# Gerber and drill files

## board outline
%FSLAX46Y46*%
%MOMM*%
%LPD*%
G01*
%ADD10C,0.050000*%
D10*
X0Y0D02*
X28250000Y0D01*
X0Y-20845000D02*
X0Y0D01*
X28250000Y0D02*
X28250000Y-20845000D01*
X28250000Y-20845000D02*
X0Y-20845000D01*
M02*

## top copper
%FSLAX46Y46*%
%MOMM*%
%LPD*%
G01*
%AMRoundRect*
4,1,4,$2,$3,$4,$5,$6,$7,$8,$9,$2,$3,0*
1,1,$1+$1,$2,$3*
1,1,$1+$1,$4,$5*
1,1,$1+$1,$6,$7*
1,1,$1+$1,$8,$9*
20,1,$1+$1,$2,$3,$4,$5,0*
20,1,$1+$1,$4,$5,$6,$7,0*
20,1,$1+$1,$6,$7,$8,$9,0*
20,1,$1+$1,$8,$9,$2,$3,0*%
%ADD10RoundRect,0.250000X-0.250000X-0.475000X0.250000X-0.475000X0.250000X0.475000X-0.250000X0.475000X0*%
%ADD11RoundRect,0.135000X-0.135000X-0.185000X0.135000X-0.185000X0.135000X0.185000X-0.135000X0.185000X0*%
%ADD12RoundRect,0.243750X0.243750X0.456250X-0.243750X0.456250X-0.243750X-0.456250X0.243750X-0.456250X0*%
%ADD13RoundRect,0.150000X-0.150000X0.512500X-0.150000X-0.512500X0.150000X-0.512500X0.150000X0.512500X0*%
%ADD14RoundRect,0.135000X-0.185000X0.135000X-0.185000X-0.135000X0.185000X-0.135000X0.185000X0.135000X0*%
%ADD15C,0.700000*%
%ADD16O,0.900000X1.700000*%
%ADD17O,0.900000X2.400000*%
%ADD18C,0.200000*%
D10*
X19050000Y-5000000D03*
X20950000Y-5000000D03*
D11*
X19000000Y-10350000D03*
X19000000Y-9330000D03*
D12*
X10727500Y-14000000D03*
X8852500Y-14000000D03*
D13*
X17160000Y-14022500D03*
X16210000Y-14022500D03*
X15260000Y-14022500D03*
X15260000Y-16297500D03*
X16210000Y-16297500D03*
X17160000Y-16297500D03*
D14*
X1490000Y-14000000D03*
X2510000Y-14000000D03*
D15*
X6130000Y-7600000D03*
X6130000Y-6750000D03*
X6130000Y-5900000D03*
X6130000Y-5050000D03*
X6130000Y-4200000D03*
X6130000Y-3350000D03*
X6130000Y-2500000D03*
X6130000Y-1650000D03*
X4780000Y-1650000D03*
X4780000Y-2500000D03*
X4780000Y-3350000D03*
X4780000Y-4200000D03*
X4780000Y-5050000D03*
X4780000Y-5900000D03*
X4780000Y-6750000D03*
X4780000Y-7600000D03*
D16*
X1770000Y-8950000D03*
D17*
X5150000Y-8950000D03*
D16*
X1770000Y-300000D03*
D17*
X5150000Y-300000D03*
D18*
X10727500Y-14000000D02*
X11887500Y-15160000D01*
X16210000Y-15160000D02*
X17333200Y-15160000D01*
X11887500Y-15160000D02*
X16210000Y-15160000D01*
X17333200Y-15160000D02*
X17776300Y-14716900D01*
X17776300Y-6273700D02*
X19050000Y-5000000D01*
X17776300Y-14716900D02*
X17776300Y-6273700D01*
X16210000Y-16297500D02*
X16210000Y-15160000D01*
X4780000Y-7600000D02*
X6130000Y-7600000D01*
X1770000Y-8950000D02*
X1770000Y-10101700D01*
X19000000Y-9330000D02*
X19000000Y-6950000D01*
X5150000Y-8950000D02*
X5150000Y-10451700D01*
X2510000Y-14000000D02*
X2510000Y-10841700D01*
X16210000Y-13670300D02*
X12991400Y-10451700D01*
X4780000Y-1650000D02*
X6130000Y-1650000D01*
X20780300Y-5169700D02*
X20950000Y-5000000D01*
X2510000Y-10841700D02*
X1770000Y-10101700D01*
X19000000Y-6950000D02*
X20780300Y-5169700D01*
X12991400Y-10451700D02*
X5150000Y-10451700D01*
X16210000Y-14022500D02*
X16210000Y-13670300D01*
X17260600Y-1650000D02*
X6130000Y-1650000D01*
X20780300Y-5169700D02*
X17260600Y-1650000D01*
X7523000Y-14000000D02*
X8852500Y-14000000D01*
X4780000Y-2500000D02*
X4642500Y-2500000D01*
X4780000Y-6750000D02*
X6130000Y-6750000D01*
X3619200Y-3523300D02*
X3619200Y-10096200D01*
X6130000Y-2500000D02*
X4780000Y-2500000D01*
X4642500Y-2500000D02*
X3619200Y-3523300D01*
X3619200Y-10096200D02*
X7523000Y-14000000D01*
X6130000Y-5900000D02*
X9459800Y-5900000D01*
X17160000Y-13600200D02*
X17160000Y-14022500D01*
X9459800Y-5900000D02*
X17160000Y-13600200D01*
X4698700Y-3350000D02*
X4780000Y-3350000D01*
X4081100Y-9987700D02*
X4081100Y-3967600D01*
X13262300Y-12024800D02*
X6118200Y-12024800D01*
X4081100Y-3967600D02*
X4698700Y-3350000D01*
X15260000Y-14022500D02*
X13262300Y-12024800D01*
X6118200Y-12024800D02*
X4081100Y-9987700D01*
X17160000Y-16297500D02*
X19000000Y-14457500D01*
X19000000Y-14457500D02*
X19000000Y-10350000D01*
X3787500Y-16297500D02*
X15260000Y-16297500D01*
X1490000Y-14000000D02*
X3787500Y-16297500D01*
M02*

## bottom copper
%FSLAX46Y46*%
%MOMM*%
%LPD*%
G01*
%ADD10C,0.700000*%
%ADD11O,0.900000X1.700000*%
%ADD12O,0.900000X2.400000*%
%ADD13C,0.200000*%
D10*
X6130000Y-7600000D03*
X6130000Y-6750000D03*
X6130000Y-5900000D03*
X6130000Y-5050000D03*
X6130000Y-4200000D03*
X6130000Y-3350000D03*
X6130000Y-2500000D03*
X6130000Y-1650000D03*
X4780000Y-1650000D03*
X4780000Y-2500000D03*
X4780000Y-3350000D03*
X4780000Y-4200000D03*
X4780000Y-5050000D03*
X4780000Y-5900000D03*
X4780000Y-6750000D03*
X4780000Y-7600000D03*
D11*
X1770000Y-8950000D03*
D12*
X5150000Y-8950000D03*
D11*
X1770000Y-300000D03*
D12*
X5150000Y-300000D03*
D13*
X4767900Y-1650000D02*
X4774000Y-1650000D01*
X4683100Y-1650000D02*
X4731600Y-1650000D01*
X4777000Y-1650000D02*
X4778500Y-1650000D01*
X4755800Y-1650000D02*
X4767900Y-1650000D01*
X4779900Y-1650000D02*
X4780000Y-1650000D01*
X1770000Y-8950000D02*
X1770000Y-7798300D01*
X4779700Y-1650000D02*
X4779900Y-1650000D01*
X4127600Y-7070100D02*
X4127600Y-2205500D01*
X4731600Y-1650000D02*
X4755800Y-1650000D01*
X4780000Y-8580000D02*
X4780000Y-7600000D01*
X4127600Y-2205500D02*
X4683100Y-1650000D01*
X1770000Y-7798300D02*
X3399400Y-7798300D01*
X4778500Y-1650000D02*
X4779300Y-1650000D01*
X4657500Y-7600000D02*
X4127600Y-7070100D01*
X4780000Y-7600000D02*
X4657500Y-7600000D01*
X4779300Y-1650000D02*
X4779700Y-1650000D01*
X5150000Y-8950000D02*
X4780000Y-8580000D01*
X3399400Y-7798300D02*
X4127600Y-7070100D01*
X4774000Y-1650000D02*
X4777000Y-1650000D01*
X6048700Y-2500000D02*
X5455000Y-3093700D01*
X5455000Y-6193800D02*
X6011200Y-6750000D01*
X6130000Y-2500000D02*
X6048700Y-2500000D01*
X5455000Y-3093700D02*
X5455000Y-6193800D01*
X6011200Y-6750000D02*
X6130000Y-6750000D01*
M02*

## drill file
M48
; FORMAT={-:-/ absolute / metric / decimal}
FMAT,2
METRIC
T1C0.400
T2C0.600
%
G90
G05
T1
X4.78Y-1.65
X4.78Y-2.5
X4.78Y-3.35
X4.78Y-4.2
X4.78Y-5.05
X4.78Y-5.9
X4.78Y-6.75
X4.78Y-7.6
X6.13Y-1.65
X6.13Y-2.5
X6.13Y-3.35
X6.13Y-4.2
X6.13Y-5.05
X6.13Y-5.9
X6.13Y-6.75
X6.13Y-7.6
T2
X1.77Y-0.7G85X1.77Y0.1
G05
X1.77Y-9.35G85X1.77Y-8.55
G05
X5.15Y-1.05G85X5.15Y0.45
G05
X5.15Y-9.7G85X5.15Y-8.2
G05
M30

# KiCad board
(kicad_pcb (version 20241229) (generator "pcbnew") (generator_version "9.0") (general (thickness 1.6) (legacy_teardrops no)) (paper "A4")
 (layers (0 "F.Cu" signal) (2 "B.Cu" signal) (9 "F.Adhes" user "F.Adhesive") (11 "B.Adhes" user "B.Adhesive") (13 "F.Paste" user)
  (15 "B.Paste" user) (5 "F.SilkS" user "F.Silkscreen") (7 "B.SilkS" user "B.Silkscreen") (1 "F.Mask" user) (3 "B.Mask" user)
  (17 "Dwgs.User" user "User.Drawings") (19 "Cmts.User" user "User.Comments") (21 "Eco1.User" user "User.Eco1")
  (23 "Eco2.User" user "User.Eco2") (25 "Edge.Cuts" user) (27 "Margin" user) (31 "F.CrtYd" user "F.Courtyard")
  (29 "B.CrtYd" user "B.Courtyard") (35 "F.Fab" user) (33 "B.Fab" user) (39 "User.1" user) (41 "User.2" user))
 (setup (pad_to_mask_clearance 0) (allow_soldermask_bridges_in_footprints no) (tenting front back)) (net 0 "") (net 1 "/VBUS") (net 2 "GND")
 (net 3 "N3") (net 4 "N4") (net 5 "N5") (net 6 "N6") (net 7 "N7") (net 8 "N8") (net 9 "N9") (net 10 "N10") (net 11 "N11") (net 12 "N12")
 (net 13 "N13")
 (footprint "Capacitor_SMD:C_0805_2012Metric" (layer "F.Cu") (at 20 5)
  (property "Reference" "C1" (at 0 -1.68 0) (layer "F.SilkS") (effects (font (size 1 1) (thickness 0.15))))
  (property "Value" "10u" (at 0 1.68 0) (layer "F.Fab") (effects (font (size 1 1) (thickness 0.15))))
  (pad "1" smd roundrect (at -0.95 0) (size 1 1.45) (layers "F.Cu" "F.Mask" "F.Paste") (roundrect_rratio 0.25) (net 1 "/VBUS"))
  (pad "2" smd roundrect (at 0.95 0) (size 1 1.45) (layers "F.Cu" "F.Mask" "F.Paste") (roundrect_rratio 0.25) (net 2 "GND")))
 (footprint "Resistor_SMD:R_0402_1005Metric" (layer "F.Cu") (at 19 9.84 90)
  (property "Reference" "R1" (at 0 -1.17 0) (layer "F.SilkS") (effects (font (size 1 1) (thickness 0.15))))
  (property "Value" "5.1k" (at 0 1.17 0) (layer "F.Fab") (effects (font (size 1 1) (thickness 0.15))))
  (pad "1" smd roundrect (at -0.51 0) (size 0.54 0.64) (layers "F.Cu" "F.Mask" "F.Paste") (roundrect_rratio 0.25) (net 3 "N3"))
  (pad "2" smd roundrect (at 0.51 0) (size 0.54 0.64) (layers "F.Cu" "F.Mask" "F.Paste") (roundrect_rratio 0.25) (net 2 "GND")))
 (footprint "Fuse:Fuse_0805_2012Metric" (layer "F.Cu") (at 9.79 14 180)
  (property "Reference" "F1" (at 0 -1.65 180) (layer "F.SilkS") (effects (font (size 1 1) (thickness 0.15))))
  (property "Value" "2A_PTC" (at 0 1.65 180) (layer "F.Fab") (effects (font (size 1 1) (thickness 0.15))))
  (pad "1" smd roundrect (at -0.9375 0 180) (size 0.975 1.4) (layers "F.Cu" "F.Mask" "F.Paste") (roundrect_rratio 0.25) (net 1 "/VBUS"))
  (pad "2" smd roundrect (at 0.9375 0 180) (size 0.975 1.4) (layers "F.Cu" "F.Mask" "F.Paste") (roundrect_rratio 0.25) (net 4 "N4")))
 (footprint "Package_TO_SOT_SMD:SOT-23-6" (layer "F.Cu") (at 16.21 15.16 -90)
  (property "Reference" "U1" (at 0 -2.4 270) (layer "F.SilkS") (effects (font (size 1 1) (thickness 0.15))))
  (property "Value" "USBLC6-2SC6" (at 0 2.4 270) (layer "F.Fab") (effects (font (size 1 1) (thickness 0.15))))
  (pad "1" smd roundrect (at -1.1375 -0.95 270) (size 1.325 0.6) (layers "F.Cu" "F.Mask" "F.Paste") (roundrect_rratio 0.25) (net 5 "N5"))
  (pad "2" smd roundrect (at -1.1375 0 270) (size 1.325 0.6) (layers "F.Cu" "F.Mask" "F.Paste") (roundrect_rratio 0.25) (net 2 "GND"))
  (pad "3" smd roundrect (at -1.1375 0.95 270) (size 1.325 0.6) (layers "F.Cu" "F.Mask" "F.Paste") (roundrect_rratio 0.25) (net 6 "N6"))
  (pad "4" smd roundrect (at 1.1375 0.95 270) (size 1.325 0.6) (layers "F.Cu" "F.Mask" "F.Paste") (roundrect_rratio 0.25) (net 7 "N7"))
  (pad "5" smd roundrect (at 1.1375 0 270) (size 1.325 0.6) (layers "F.Cu" "F.Mask" "F.Paste") (roundrect_rratio 0.25) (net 1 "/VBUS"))
  (pad "6" smd roundrect (at 1.1375 -0.95 270) (size 1.325 0.6) (layers "F.Cu" "F.Mask" "F.Paste") (roundrect_rratio 0.25) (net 3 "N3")))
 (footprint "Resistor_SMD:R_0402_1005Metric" (layer "F.Cu") (at 2 14)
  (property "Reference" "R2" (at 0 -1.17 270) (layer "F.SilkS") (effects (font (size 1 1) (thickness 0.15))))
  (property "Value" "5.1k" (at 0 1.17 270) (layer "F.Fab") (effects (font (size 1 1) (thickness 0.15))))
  (pad "1" smd roundrect (at -0.51 0 270) (size 0.54 0.64) (layers "F.Cu" "F.Mask" "F.Paste") (roundrect_rratio 0.25) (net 7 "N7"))
  (pad "2" smd roundrect (at 0.51 0 270) (size 0.54 0.64) (layers "F.Cu" "F.Mask" "F.Paste") (roundrect_rratio 0.25) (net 2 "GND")))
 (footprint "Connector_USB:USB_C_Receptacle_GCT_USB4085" (layer "B.Cu") (at 6.13 7.6 90)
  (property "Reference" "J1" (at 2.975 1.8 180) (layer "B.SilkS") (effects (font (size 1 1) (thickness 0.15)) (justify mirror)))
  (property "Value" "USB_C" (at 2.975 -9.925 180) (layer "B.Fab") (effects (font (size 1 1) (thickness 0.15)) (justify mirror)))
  (pad "A1" thru_hole circle (at 0 0 180) (size 0.7 0.7) (drill 0.4) (layers "*.Cu" "*.Mask") (remove_unused_layers no) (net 2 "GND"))
  (pad "A4" thru_hole circle (at 0.85 0 180) (size 0.7 0.7) (drill 0.4) (layers "*.Cu" "*.Mask") (remove_unused_layers no) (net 4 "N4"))
  (pad "A5" thru_hole circle (at 1.7 0 180) (size 0.7 0.7) (drill 0.4) (layers "*.Cu" "*.Mask") (remove_unused_layers no) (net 5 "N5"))
  (pad "A6" thru_hole circle (at 2.55 0 180) (size 0.7 0.7) (drill 0.4) (layers "*.Cu" "*.Mask") (remove_unused_layers no) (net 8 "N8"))
  (pad "A7" thru_hole circle (at 3.4 0 180) (size 0.7 0.7) (drill 0.4) (layers "*.Cu" "*.Mask") (remove_unused_layers no) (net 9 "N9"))
  (pad "A8" thru_hole circle (at 4.25 0 180) (size 0.7 0.7) (drill 0.4) (layers "*.Cu" "*.Mask") (remove_unused_layers no) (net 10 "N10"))
  (pad "A9" thru_hole circle (at 5.1 0 180) (size 0.7 0.7) (drill 0.4) (layers "*.Cu" "*.Mask") (remove_unused_layers no) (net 4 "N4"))
  (pad "A12" thru_hole circle (at 5.95 0 180) (size 0.7 0.7) (drill 0.4) (layers "*.Cu" "*.Mask") (remove_unused_layers no) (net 2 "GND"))
  (pad "B1" thru_hole circle (at 5.95 -1.35 180) (size 0.7 0.7) (drill 0.4) (layers "*.Cu" "*.Mask") (remove_unused_layers no) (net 2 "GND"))
  (pad "B4" thru_hole circle (at 5.1 -1.35 180) (size 0.7 0.7) (drill 0.4) (layers "*.Cu" "*.Mask") (remove_unused_layers no) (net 4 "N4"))
  (pad "B5" thru_hole circle (at 4.25 -1.35 180) (size 0.7 0.7) (drill 0.4) (layers "*.Cu" "*.Mask") (remove_unused_layers no) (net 6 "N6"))
  (pad "B6" thru_hole circle (at 3.4 -1.35 180) (size 0.7 0.7) (drill 0.4) (layers "*.Cu" "*.Mask") (remove_unused_layers no) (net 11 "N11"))
  (pad "B7" thru_hole circle (at 2.55 -1.35 180) (size 0.7 0.7) (drill 0.4) (layers "*.Cu" "*.Mask") (remove_unused_layers no)
   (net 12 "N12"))
  (pad "B8" thru_hole circle (at 1.7 -1.35 180) (size 0.7 0.7) (drill 0.4) (layers "*.Cu" "*.Mask") (remove_unused_layers no) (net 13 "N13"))
  (pad "B9" thru_hole circle (at 0.85 -1.35 180) (size 0.7 0.7) (drill 0.4) (layers "*.Cu" "*.Mask") (remove_unused_layers no) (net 4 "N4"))
  (pad "B12" thru_hole circle (at 0 -1.35 180) (size 0.7 0.7) (drill 0.4) (layers "*.Cu" "*.Mask") (remove_unused_layers no) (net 2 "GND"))
  (pad "S1" thru_hole oval (at -1.35 -4.36 180) (size 0.9 1.7) (drill oval 0.6 1.4) (layers "*.Cu" "*.Mask") (remove_unused_layers no)
   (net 2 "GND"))
  (pad "S1" thru_hole oval (at -1.35 -0.98 180) (size 0.9 2.4) (drill oval 0.6 2.1) (layers "*.Cu" "*.Mask") (remove_unused_layers no)
   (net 2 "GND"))
  (pad "S1" thru_hole oval (at 7.3 -4.36 180) (size 0.9 1.7) (drill oval 0.6 1.4) (layers "*.Cu" "*.Mask") (remove_unused_layers no)
   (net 2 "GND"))
  (pad "S1" thru_hole oval (at 7.3 -0.98 180) (size 0.9 2.4) (drill oval 0.6 2.1) (layers "*.Cu" "*.Mask") (remove_unused_layers no)
   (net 2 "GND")))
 (gr_line (start 0 0) (end 28.25 0) (stroke (width 0.05) (type default)) (layer "Edge.Cuts"))
 (gr_line (start 0 20.845) (end 0 0) (stroke (width 0.05) (type default)) (layer "Edge.Cuts"))
 (gr_line (start 28.25 0) (end 28.25 20.845) (stroke (width 0.05) (type default)) (layer "Edge.Cuts"))
 (gr_line (start 28.25 20.845) (end 0 20.845) (stroke (width 0.05) (type default)) (layer "Edge.Cuts"))
 (segment (start 10.7275 14) (end 11.8875 15.16) (width 0.2) (layer "F.Cu") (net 1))
 (segment (start 16.21 15.16) (end 17.3332 15.16) (width 0.2) (layer "F.Cu") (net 1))
 (segment (start 11.8875 15.16) (end 16.21 15.16) (width 0.2) (layer "F.Cu") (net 1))
 (segment (start 17.3332 15.16) (end 17.7763 14.7169) (width 0.2) (layer "F.Cu") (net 1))
 (segment (start 17.7763 6.2737) (end 19.05 5) (width 0.2) (layer "F.Cu") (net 1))
 (segment (start 17.7763 14.7169) (end 17.7763 6.2737) (width 0.2) (layer "F.Cu") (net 1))
 (segment (start 16.21 16.2975) (end 16.21 15.16) (width 0.2) (layer "F.Cu") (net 1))
 (segment (start 4.78 7.6) (end 6.13 7.6) (width 0.2) (layer "F.Cu") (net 2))
 (segment (start 1.77 8.95) (end 1.77 10.1017) (width 0.2) (layer "F.Cu") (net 2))
 (segment (start 19 9.33) (end 19 6.95) (width 0.2) (layer "F.Cu") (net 2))
 (segment (start 5.15 8.95) (end 5.15 10.4517) (width 0.2) (layer "F.Cu") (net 2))
 (segment (start 2.51 14) (end 2.51 10.8417) (width 0.2) (layer "F.Cu") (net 2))
 (segment (start 16.21 13.6703) (end 12.9914 10.4517) (width 0.2) (layer "F.Cu") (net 2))
 (segment (start 4.78 1.65) (end 6.13 1.65) (width 0.2) (layer "F.Cu") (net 2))
 (segment (start 20.7803 5.1697) (end 20.95 5) (width 0.2) (layer "F.Cu") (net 2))
 (segment (start 2.51 10.8417) (end 1.77 10.1017) (width 0.2) (layer "F.Cu") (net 2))
 (segment (start 19 6.95) (end 20.7803 5.1697) (width 0.2) (layer "F.Cu") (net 2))
 (segment (start 12.9914 10.4517) (end 5.15 10.4517) (width 0.2) (layer "F.Cu") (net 2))
 (segment (start 16.21 14.0225) (end 16.21 13.6703) (width 0.2) (layer "F.Cu") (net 2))
 (segment (start 17.2606 1.65) (end 6.13 1.65) (width 0.2) (layer "F.Cu") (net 2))
 (segment (start 20.7803 5.1697) (end 17.2606 1.65) (width 0.2) (layer "F.Cu") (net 2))
 (segment (start 4.7679 1.65) (end 4.774 1.65) (width 0.2) (layer "B.Cu") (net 2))
 (segment (start 4.6831 1.65) (end 4.7316 1.65) (width 0.2) (layer "B.Cu") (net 2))
 (segment (start 4.777 1.65) (end 4.7785 1.65) (width 0.2) (layer "B.Cu") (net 2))
 (segment (start 4.7558 1.65) (end 4.7679 1.65) (width 0.2) (layer "B.Cu") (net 2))
 (segment (start 4.7799 1.65) (end 4.78 1.65) (width 0.2) (layer "B.Cu") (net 2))
 (segment (start 1.77 8.95) (end 1.77 7.7983) (width 0.2) (layer "B.Cu") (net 2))
 (segment (start 4.7797 1.65) (end 4.7799 1.65) (width 0.2) (layer "B.Cu") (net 2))
 (segment (start 4.1276 7.0701) (end 4.1276 2.2055) (width 0.2) (layer "B.Cu") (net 2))
 (segment (start 4.7316 1.65) (end 4.7558 1.65) (width 0.2) (layer "B.Cu") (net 2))
 (segment (start 4.78 8.58) (end 4.78 7.6) (width 0.2) (layer "B.Cu") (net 2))
 (segment (start 4.1276 2.2055) (end 4.6831 1.65) (width 0.2) (layer "B.Cu") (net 2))
 (segment (start 1.77 7.7983) (end 3.3994 7.7983) (width 0.2) (layer "B.Cu") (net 2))
 (segment (start 4.7785 1.65) (end 4.7793 1.65) (width 0.2) (layer "B.Cu") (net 2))
 (segment (start 4.6575 7.6) (end 4.1276 7.0701) (width 0.2) (layer "B.Cu") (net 2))
 (segment (start 4.78 7.6) (end 4.6575 7.6) (width 0.2) (layer "B.Cu") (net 2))
 (segment (start 4.7793 1.65) (end 4.7797 1.65) (width 0.2) (layer "B.Cu") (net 2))
 (segment (start 5.15 8.95) (end 4.78 8.58) (width 0.2) (layer "B.Cu") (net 2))
 (segment (start 3.3994 7.7983) (end 4.1276 7.0701) (width 0.2) (layer "B.Cu") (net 2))
 (segment (start 4.774 1.65) (end 4.777 1.65) (width 0.2) (layer "B.Cu") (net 2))
 (segment (start 7.523 14) (end 8.8525 14) (width 0.2) (layer "F.Cu") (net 4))
 (segment (start 4.78 2.5) (end 4.6425 2.5) (width 0.2) (layer "F.Cu") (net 4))
 (segment (start 4.78 6.75) (end 6.13 6.75) (width 0.2) (layer "F.Cu") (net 4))
 (segment (start 3.6192 3.5233) (end 3.6192 10.0962) (width 0.2) (layer "F.Cu") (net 4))
 (segment (start 6.13 2.5) (end 4.78 2.5) (width 0.2) (layer "F.Cu") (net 4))
 (segment (start 4.6425 2.5) (end 3.6192 3.5233) (width 0.2) (layer "F.Cu") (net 4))
 (segment (start 3.6192 10.0962) (end 7.523 14) (width 0.2) (layer "F.Cu") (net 4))
 (segment (start 6.0487 2.5) (end 5.455 3.0937) (width 0.2) (layer "B.Cu") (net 4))
 (segment (start 5.455 6.1938) (end 6.0112 6.75) (width 0.2) (layer "B.Cu") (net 4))
 (segment (start 6.13 2.5) (end 6.0487 2.5) (width 0.2) (layer "B.Cu") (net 4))
 (segment (start 5.455 3.0937) (end 5.455 6.1938) (width 0.2) (layer "B.Cu") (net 4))
 (segment (start 6.0112 6.75) (end 6.13 6.75) (width 0.2) (layer "B.Cu") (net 4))
 (segment (start 6.13 5.9) (end 9.4598 5.9) (width 0.2) (layer "F.Cu") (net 5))
 (segment (start 17.16 13.6002) (end 17.16 14.0225) (width 0.2) (layer "F.Cu") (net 5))
 (segment (start 9.4598 5.9) (end 17.16 13.6002) (width 0.2) (layer "F.Cu") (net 5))
 (segment (start 4.6987 3.35) (end 4.78 3.35) (width 0.2) (layer "F.Cu") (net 6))
 (segment (start 4.0811 9.9877) (end 4.0811 3.9676) (width 0.2) (layer "F.Cu") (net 6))
 (segment (start 13.2623 12.0248) (end 6.1182 12.0248) (width 0.2) (layer "F.Cu") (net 6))
 (segment (start 4.0811 3.9676) (end 4.6987 3.35) (width 0.2) (layer "F.Cu") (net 6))
 (segment (start 15.26 14.0225) (end 13.2623 12.0248) (width 0.2) (layer "F.Cu") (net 6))
 (segment (start 6.1182 12.0248) (end 4.0811 9.9877) (width 0.2) (layer "F.Cu") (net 6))
 (segment (start 17.16 16.2975) (end 19 14.4575) (width 0.2) (layer "F.Cu") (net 3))
 (segment (start 19 14.4575) (end 19 10.35) (width 0.2) (layer "F.Cu") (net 3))
 (segment (start 3.7875 16.2975) (end 15.26 16.2975) (width 0.2) (layer "F.Cu") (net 7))
 (segment (start 1.49 14) (end 3.7875 16.2975) (width 0.2) (layer "F.Cu") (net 7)))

